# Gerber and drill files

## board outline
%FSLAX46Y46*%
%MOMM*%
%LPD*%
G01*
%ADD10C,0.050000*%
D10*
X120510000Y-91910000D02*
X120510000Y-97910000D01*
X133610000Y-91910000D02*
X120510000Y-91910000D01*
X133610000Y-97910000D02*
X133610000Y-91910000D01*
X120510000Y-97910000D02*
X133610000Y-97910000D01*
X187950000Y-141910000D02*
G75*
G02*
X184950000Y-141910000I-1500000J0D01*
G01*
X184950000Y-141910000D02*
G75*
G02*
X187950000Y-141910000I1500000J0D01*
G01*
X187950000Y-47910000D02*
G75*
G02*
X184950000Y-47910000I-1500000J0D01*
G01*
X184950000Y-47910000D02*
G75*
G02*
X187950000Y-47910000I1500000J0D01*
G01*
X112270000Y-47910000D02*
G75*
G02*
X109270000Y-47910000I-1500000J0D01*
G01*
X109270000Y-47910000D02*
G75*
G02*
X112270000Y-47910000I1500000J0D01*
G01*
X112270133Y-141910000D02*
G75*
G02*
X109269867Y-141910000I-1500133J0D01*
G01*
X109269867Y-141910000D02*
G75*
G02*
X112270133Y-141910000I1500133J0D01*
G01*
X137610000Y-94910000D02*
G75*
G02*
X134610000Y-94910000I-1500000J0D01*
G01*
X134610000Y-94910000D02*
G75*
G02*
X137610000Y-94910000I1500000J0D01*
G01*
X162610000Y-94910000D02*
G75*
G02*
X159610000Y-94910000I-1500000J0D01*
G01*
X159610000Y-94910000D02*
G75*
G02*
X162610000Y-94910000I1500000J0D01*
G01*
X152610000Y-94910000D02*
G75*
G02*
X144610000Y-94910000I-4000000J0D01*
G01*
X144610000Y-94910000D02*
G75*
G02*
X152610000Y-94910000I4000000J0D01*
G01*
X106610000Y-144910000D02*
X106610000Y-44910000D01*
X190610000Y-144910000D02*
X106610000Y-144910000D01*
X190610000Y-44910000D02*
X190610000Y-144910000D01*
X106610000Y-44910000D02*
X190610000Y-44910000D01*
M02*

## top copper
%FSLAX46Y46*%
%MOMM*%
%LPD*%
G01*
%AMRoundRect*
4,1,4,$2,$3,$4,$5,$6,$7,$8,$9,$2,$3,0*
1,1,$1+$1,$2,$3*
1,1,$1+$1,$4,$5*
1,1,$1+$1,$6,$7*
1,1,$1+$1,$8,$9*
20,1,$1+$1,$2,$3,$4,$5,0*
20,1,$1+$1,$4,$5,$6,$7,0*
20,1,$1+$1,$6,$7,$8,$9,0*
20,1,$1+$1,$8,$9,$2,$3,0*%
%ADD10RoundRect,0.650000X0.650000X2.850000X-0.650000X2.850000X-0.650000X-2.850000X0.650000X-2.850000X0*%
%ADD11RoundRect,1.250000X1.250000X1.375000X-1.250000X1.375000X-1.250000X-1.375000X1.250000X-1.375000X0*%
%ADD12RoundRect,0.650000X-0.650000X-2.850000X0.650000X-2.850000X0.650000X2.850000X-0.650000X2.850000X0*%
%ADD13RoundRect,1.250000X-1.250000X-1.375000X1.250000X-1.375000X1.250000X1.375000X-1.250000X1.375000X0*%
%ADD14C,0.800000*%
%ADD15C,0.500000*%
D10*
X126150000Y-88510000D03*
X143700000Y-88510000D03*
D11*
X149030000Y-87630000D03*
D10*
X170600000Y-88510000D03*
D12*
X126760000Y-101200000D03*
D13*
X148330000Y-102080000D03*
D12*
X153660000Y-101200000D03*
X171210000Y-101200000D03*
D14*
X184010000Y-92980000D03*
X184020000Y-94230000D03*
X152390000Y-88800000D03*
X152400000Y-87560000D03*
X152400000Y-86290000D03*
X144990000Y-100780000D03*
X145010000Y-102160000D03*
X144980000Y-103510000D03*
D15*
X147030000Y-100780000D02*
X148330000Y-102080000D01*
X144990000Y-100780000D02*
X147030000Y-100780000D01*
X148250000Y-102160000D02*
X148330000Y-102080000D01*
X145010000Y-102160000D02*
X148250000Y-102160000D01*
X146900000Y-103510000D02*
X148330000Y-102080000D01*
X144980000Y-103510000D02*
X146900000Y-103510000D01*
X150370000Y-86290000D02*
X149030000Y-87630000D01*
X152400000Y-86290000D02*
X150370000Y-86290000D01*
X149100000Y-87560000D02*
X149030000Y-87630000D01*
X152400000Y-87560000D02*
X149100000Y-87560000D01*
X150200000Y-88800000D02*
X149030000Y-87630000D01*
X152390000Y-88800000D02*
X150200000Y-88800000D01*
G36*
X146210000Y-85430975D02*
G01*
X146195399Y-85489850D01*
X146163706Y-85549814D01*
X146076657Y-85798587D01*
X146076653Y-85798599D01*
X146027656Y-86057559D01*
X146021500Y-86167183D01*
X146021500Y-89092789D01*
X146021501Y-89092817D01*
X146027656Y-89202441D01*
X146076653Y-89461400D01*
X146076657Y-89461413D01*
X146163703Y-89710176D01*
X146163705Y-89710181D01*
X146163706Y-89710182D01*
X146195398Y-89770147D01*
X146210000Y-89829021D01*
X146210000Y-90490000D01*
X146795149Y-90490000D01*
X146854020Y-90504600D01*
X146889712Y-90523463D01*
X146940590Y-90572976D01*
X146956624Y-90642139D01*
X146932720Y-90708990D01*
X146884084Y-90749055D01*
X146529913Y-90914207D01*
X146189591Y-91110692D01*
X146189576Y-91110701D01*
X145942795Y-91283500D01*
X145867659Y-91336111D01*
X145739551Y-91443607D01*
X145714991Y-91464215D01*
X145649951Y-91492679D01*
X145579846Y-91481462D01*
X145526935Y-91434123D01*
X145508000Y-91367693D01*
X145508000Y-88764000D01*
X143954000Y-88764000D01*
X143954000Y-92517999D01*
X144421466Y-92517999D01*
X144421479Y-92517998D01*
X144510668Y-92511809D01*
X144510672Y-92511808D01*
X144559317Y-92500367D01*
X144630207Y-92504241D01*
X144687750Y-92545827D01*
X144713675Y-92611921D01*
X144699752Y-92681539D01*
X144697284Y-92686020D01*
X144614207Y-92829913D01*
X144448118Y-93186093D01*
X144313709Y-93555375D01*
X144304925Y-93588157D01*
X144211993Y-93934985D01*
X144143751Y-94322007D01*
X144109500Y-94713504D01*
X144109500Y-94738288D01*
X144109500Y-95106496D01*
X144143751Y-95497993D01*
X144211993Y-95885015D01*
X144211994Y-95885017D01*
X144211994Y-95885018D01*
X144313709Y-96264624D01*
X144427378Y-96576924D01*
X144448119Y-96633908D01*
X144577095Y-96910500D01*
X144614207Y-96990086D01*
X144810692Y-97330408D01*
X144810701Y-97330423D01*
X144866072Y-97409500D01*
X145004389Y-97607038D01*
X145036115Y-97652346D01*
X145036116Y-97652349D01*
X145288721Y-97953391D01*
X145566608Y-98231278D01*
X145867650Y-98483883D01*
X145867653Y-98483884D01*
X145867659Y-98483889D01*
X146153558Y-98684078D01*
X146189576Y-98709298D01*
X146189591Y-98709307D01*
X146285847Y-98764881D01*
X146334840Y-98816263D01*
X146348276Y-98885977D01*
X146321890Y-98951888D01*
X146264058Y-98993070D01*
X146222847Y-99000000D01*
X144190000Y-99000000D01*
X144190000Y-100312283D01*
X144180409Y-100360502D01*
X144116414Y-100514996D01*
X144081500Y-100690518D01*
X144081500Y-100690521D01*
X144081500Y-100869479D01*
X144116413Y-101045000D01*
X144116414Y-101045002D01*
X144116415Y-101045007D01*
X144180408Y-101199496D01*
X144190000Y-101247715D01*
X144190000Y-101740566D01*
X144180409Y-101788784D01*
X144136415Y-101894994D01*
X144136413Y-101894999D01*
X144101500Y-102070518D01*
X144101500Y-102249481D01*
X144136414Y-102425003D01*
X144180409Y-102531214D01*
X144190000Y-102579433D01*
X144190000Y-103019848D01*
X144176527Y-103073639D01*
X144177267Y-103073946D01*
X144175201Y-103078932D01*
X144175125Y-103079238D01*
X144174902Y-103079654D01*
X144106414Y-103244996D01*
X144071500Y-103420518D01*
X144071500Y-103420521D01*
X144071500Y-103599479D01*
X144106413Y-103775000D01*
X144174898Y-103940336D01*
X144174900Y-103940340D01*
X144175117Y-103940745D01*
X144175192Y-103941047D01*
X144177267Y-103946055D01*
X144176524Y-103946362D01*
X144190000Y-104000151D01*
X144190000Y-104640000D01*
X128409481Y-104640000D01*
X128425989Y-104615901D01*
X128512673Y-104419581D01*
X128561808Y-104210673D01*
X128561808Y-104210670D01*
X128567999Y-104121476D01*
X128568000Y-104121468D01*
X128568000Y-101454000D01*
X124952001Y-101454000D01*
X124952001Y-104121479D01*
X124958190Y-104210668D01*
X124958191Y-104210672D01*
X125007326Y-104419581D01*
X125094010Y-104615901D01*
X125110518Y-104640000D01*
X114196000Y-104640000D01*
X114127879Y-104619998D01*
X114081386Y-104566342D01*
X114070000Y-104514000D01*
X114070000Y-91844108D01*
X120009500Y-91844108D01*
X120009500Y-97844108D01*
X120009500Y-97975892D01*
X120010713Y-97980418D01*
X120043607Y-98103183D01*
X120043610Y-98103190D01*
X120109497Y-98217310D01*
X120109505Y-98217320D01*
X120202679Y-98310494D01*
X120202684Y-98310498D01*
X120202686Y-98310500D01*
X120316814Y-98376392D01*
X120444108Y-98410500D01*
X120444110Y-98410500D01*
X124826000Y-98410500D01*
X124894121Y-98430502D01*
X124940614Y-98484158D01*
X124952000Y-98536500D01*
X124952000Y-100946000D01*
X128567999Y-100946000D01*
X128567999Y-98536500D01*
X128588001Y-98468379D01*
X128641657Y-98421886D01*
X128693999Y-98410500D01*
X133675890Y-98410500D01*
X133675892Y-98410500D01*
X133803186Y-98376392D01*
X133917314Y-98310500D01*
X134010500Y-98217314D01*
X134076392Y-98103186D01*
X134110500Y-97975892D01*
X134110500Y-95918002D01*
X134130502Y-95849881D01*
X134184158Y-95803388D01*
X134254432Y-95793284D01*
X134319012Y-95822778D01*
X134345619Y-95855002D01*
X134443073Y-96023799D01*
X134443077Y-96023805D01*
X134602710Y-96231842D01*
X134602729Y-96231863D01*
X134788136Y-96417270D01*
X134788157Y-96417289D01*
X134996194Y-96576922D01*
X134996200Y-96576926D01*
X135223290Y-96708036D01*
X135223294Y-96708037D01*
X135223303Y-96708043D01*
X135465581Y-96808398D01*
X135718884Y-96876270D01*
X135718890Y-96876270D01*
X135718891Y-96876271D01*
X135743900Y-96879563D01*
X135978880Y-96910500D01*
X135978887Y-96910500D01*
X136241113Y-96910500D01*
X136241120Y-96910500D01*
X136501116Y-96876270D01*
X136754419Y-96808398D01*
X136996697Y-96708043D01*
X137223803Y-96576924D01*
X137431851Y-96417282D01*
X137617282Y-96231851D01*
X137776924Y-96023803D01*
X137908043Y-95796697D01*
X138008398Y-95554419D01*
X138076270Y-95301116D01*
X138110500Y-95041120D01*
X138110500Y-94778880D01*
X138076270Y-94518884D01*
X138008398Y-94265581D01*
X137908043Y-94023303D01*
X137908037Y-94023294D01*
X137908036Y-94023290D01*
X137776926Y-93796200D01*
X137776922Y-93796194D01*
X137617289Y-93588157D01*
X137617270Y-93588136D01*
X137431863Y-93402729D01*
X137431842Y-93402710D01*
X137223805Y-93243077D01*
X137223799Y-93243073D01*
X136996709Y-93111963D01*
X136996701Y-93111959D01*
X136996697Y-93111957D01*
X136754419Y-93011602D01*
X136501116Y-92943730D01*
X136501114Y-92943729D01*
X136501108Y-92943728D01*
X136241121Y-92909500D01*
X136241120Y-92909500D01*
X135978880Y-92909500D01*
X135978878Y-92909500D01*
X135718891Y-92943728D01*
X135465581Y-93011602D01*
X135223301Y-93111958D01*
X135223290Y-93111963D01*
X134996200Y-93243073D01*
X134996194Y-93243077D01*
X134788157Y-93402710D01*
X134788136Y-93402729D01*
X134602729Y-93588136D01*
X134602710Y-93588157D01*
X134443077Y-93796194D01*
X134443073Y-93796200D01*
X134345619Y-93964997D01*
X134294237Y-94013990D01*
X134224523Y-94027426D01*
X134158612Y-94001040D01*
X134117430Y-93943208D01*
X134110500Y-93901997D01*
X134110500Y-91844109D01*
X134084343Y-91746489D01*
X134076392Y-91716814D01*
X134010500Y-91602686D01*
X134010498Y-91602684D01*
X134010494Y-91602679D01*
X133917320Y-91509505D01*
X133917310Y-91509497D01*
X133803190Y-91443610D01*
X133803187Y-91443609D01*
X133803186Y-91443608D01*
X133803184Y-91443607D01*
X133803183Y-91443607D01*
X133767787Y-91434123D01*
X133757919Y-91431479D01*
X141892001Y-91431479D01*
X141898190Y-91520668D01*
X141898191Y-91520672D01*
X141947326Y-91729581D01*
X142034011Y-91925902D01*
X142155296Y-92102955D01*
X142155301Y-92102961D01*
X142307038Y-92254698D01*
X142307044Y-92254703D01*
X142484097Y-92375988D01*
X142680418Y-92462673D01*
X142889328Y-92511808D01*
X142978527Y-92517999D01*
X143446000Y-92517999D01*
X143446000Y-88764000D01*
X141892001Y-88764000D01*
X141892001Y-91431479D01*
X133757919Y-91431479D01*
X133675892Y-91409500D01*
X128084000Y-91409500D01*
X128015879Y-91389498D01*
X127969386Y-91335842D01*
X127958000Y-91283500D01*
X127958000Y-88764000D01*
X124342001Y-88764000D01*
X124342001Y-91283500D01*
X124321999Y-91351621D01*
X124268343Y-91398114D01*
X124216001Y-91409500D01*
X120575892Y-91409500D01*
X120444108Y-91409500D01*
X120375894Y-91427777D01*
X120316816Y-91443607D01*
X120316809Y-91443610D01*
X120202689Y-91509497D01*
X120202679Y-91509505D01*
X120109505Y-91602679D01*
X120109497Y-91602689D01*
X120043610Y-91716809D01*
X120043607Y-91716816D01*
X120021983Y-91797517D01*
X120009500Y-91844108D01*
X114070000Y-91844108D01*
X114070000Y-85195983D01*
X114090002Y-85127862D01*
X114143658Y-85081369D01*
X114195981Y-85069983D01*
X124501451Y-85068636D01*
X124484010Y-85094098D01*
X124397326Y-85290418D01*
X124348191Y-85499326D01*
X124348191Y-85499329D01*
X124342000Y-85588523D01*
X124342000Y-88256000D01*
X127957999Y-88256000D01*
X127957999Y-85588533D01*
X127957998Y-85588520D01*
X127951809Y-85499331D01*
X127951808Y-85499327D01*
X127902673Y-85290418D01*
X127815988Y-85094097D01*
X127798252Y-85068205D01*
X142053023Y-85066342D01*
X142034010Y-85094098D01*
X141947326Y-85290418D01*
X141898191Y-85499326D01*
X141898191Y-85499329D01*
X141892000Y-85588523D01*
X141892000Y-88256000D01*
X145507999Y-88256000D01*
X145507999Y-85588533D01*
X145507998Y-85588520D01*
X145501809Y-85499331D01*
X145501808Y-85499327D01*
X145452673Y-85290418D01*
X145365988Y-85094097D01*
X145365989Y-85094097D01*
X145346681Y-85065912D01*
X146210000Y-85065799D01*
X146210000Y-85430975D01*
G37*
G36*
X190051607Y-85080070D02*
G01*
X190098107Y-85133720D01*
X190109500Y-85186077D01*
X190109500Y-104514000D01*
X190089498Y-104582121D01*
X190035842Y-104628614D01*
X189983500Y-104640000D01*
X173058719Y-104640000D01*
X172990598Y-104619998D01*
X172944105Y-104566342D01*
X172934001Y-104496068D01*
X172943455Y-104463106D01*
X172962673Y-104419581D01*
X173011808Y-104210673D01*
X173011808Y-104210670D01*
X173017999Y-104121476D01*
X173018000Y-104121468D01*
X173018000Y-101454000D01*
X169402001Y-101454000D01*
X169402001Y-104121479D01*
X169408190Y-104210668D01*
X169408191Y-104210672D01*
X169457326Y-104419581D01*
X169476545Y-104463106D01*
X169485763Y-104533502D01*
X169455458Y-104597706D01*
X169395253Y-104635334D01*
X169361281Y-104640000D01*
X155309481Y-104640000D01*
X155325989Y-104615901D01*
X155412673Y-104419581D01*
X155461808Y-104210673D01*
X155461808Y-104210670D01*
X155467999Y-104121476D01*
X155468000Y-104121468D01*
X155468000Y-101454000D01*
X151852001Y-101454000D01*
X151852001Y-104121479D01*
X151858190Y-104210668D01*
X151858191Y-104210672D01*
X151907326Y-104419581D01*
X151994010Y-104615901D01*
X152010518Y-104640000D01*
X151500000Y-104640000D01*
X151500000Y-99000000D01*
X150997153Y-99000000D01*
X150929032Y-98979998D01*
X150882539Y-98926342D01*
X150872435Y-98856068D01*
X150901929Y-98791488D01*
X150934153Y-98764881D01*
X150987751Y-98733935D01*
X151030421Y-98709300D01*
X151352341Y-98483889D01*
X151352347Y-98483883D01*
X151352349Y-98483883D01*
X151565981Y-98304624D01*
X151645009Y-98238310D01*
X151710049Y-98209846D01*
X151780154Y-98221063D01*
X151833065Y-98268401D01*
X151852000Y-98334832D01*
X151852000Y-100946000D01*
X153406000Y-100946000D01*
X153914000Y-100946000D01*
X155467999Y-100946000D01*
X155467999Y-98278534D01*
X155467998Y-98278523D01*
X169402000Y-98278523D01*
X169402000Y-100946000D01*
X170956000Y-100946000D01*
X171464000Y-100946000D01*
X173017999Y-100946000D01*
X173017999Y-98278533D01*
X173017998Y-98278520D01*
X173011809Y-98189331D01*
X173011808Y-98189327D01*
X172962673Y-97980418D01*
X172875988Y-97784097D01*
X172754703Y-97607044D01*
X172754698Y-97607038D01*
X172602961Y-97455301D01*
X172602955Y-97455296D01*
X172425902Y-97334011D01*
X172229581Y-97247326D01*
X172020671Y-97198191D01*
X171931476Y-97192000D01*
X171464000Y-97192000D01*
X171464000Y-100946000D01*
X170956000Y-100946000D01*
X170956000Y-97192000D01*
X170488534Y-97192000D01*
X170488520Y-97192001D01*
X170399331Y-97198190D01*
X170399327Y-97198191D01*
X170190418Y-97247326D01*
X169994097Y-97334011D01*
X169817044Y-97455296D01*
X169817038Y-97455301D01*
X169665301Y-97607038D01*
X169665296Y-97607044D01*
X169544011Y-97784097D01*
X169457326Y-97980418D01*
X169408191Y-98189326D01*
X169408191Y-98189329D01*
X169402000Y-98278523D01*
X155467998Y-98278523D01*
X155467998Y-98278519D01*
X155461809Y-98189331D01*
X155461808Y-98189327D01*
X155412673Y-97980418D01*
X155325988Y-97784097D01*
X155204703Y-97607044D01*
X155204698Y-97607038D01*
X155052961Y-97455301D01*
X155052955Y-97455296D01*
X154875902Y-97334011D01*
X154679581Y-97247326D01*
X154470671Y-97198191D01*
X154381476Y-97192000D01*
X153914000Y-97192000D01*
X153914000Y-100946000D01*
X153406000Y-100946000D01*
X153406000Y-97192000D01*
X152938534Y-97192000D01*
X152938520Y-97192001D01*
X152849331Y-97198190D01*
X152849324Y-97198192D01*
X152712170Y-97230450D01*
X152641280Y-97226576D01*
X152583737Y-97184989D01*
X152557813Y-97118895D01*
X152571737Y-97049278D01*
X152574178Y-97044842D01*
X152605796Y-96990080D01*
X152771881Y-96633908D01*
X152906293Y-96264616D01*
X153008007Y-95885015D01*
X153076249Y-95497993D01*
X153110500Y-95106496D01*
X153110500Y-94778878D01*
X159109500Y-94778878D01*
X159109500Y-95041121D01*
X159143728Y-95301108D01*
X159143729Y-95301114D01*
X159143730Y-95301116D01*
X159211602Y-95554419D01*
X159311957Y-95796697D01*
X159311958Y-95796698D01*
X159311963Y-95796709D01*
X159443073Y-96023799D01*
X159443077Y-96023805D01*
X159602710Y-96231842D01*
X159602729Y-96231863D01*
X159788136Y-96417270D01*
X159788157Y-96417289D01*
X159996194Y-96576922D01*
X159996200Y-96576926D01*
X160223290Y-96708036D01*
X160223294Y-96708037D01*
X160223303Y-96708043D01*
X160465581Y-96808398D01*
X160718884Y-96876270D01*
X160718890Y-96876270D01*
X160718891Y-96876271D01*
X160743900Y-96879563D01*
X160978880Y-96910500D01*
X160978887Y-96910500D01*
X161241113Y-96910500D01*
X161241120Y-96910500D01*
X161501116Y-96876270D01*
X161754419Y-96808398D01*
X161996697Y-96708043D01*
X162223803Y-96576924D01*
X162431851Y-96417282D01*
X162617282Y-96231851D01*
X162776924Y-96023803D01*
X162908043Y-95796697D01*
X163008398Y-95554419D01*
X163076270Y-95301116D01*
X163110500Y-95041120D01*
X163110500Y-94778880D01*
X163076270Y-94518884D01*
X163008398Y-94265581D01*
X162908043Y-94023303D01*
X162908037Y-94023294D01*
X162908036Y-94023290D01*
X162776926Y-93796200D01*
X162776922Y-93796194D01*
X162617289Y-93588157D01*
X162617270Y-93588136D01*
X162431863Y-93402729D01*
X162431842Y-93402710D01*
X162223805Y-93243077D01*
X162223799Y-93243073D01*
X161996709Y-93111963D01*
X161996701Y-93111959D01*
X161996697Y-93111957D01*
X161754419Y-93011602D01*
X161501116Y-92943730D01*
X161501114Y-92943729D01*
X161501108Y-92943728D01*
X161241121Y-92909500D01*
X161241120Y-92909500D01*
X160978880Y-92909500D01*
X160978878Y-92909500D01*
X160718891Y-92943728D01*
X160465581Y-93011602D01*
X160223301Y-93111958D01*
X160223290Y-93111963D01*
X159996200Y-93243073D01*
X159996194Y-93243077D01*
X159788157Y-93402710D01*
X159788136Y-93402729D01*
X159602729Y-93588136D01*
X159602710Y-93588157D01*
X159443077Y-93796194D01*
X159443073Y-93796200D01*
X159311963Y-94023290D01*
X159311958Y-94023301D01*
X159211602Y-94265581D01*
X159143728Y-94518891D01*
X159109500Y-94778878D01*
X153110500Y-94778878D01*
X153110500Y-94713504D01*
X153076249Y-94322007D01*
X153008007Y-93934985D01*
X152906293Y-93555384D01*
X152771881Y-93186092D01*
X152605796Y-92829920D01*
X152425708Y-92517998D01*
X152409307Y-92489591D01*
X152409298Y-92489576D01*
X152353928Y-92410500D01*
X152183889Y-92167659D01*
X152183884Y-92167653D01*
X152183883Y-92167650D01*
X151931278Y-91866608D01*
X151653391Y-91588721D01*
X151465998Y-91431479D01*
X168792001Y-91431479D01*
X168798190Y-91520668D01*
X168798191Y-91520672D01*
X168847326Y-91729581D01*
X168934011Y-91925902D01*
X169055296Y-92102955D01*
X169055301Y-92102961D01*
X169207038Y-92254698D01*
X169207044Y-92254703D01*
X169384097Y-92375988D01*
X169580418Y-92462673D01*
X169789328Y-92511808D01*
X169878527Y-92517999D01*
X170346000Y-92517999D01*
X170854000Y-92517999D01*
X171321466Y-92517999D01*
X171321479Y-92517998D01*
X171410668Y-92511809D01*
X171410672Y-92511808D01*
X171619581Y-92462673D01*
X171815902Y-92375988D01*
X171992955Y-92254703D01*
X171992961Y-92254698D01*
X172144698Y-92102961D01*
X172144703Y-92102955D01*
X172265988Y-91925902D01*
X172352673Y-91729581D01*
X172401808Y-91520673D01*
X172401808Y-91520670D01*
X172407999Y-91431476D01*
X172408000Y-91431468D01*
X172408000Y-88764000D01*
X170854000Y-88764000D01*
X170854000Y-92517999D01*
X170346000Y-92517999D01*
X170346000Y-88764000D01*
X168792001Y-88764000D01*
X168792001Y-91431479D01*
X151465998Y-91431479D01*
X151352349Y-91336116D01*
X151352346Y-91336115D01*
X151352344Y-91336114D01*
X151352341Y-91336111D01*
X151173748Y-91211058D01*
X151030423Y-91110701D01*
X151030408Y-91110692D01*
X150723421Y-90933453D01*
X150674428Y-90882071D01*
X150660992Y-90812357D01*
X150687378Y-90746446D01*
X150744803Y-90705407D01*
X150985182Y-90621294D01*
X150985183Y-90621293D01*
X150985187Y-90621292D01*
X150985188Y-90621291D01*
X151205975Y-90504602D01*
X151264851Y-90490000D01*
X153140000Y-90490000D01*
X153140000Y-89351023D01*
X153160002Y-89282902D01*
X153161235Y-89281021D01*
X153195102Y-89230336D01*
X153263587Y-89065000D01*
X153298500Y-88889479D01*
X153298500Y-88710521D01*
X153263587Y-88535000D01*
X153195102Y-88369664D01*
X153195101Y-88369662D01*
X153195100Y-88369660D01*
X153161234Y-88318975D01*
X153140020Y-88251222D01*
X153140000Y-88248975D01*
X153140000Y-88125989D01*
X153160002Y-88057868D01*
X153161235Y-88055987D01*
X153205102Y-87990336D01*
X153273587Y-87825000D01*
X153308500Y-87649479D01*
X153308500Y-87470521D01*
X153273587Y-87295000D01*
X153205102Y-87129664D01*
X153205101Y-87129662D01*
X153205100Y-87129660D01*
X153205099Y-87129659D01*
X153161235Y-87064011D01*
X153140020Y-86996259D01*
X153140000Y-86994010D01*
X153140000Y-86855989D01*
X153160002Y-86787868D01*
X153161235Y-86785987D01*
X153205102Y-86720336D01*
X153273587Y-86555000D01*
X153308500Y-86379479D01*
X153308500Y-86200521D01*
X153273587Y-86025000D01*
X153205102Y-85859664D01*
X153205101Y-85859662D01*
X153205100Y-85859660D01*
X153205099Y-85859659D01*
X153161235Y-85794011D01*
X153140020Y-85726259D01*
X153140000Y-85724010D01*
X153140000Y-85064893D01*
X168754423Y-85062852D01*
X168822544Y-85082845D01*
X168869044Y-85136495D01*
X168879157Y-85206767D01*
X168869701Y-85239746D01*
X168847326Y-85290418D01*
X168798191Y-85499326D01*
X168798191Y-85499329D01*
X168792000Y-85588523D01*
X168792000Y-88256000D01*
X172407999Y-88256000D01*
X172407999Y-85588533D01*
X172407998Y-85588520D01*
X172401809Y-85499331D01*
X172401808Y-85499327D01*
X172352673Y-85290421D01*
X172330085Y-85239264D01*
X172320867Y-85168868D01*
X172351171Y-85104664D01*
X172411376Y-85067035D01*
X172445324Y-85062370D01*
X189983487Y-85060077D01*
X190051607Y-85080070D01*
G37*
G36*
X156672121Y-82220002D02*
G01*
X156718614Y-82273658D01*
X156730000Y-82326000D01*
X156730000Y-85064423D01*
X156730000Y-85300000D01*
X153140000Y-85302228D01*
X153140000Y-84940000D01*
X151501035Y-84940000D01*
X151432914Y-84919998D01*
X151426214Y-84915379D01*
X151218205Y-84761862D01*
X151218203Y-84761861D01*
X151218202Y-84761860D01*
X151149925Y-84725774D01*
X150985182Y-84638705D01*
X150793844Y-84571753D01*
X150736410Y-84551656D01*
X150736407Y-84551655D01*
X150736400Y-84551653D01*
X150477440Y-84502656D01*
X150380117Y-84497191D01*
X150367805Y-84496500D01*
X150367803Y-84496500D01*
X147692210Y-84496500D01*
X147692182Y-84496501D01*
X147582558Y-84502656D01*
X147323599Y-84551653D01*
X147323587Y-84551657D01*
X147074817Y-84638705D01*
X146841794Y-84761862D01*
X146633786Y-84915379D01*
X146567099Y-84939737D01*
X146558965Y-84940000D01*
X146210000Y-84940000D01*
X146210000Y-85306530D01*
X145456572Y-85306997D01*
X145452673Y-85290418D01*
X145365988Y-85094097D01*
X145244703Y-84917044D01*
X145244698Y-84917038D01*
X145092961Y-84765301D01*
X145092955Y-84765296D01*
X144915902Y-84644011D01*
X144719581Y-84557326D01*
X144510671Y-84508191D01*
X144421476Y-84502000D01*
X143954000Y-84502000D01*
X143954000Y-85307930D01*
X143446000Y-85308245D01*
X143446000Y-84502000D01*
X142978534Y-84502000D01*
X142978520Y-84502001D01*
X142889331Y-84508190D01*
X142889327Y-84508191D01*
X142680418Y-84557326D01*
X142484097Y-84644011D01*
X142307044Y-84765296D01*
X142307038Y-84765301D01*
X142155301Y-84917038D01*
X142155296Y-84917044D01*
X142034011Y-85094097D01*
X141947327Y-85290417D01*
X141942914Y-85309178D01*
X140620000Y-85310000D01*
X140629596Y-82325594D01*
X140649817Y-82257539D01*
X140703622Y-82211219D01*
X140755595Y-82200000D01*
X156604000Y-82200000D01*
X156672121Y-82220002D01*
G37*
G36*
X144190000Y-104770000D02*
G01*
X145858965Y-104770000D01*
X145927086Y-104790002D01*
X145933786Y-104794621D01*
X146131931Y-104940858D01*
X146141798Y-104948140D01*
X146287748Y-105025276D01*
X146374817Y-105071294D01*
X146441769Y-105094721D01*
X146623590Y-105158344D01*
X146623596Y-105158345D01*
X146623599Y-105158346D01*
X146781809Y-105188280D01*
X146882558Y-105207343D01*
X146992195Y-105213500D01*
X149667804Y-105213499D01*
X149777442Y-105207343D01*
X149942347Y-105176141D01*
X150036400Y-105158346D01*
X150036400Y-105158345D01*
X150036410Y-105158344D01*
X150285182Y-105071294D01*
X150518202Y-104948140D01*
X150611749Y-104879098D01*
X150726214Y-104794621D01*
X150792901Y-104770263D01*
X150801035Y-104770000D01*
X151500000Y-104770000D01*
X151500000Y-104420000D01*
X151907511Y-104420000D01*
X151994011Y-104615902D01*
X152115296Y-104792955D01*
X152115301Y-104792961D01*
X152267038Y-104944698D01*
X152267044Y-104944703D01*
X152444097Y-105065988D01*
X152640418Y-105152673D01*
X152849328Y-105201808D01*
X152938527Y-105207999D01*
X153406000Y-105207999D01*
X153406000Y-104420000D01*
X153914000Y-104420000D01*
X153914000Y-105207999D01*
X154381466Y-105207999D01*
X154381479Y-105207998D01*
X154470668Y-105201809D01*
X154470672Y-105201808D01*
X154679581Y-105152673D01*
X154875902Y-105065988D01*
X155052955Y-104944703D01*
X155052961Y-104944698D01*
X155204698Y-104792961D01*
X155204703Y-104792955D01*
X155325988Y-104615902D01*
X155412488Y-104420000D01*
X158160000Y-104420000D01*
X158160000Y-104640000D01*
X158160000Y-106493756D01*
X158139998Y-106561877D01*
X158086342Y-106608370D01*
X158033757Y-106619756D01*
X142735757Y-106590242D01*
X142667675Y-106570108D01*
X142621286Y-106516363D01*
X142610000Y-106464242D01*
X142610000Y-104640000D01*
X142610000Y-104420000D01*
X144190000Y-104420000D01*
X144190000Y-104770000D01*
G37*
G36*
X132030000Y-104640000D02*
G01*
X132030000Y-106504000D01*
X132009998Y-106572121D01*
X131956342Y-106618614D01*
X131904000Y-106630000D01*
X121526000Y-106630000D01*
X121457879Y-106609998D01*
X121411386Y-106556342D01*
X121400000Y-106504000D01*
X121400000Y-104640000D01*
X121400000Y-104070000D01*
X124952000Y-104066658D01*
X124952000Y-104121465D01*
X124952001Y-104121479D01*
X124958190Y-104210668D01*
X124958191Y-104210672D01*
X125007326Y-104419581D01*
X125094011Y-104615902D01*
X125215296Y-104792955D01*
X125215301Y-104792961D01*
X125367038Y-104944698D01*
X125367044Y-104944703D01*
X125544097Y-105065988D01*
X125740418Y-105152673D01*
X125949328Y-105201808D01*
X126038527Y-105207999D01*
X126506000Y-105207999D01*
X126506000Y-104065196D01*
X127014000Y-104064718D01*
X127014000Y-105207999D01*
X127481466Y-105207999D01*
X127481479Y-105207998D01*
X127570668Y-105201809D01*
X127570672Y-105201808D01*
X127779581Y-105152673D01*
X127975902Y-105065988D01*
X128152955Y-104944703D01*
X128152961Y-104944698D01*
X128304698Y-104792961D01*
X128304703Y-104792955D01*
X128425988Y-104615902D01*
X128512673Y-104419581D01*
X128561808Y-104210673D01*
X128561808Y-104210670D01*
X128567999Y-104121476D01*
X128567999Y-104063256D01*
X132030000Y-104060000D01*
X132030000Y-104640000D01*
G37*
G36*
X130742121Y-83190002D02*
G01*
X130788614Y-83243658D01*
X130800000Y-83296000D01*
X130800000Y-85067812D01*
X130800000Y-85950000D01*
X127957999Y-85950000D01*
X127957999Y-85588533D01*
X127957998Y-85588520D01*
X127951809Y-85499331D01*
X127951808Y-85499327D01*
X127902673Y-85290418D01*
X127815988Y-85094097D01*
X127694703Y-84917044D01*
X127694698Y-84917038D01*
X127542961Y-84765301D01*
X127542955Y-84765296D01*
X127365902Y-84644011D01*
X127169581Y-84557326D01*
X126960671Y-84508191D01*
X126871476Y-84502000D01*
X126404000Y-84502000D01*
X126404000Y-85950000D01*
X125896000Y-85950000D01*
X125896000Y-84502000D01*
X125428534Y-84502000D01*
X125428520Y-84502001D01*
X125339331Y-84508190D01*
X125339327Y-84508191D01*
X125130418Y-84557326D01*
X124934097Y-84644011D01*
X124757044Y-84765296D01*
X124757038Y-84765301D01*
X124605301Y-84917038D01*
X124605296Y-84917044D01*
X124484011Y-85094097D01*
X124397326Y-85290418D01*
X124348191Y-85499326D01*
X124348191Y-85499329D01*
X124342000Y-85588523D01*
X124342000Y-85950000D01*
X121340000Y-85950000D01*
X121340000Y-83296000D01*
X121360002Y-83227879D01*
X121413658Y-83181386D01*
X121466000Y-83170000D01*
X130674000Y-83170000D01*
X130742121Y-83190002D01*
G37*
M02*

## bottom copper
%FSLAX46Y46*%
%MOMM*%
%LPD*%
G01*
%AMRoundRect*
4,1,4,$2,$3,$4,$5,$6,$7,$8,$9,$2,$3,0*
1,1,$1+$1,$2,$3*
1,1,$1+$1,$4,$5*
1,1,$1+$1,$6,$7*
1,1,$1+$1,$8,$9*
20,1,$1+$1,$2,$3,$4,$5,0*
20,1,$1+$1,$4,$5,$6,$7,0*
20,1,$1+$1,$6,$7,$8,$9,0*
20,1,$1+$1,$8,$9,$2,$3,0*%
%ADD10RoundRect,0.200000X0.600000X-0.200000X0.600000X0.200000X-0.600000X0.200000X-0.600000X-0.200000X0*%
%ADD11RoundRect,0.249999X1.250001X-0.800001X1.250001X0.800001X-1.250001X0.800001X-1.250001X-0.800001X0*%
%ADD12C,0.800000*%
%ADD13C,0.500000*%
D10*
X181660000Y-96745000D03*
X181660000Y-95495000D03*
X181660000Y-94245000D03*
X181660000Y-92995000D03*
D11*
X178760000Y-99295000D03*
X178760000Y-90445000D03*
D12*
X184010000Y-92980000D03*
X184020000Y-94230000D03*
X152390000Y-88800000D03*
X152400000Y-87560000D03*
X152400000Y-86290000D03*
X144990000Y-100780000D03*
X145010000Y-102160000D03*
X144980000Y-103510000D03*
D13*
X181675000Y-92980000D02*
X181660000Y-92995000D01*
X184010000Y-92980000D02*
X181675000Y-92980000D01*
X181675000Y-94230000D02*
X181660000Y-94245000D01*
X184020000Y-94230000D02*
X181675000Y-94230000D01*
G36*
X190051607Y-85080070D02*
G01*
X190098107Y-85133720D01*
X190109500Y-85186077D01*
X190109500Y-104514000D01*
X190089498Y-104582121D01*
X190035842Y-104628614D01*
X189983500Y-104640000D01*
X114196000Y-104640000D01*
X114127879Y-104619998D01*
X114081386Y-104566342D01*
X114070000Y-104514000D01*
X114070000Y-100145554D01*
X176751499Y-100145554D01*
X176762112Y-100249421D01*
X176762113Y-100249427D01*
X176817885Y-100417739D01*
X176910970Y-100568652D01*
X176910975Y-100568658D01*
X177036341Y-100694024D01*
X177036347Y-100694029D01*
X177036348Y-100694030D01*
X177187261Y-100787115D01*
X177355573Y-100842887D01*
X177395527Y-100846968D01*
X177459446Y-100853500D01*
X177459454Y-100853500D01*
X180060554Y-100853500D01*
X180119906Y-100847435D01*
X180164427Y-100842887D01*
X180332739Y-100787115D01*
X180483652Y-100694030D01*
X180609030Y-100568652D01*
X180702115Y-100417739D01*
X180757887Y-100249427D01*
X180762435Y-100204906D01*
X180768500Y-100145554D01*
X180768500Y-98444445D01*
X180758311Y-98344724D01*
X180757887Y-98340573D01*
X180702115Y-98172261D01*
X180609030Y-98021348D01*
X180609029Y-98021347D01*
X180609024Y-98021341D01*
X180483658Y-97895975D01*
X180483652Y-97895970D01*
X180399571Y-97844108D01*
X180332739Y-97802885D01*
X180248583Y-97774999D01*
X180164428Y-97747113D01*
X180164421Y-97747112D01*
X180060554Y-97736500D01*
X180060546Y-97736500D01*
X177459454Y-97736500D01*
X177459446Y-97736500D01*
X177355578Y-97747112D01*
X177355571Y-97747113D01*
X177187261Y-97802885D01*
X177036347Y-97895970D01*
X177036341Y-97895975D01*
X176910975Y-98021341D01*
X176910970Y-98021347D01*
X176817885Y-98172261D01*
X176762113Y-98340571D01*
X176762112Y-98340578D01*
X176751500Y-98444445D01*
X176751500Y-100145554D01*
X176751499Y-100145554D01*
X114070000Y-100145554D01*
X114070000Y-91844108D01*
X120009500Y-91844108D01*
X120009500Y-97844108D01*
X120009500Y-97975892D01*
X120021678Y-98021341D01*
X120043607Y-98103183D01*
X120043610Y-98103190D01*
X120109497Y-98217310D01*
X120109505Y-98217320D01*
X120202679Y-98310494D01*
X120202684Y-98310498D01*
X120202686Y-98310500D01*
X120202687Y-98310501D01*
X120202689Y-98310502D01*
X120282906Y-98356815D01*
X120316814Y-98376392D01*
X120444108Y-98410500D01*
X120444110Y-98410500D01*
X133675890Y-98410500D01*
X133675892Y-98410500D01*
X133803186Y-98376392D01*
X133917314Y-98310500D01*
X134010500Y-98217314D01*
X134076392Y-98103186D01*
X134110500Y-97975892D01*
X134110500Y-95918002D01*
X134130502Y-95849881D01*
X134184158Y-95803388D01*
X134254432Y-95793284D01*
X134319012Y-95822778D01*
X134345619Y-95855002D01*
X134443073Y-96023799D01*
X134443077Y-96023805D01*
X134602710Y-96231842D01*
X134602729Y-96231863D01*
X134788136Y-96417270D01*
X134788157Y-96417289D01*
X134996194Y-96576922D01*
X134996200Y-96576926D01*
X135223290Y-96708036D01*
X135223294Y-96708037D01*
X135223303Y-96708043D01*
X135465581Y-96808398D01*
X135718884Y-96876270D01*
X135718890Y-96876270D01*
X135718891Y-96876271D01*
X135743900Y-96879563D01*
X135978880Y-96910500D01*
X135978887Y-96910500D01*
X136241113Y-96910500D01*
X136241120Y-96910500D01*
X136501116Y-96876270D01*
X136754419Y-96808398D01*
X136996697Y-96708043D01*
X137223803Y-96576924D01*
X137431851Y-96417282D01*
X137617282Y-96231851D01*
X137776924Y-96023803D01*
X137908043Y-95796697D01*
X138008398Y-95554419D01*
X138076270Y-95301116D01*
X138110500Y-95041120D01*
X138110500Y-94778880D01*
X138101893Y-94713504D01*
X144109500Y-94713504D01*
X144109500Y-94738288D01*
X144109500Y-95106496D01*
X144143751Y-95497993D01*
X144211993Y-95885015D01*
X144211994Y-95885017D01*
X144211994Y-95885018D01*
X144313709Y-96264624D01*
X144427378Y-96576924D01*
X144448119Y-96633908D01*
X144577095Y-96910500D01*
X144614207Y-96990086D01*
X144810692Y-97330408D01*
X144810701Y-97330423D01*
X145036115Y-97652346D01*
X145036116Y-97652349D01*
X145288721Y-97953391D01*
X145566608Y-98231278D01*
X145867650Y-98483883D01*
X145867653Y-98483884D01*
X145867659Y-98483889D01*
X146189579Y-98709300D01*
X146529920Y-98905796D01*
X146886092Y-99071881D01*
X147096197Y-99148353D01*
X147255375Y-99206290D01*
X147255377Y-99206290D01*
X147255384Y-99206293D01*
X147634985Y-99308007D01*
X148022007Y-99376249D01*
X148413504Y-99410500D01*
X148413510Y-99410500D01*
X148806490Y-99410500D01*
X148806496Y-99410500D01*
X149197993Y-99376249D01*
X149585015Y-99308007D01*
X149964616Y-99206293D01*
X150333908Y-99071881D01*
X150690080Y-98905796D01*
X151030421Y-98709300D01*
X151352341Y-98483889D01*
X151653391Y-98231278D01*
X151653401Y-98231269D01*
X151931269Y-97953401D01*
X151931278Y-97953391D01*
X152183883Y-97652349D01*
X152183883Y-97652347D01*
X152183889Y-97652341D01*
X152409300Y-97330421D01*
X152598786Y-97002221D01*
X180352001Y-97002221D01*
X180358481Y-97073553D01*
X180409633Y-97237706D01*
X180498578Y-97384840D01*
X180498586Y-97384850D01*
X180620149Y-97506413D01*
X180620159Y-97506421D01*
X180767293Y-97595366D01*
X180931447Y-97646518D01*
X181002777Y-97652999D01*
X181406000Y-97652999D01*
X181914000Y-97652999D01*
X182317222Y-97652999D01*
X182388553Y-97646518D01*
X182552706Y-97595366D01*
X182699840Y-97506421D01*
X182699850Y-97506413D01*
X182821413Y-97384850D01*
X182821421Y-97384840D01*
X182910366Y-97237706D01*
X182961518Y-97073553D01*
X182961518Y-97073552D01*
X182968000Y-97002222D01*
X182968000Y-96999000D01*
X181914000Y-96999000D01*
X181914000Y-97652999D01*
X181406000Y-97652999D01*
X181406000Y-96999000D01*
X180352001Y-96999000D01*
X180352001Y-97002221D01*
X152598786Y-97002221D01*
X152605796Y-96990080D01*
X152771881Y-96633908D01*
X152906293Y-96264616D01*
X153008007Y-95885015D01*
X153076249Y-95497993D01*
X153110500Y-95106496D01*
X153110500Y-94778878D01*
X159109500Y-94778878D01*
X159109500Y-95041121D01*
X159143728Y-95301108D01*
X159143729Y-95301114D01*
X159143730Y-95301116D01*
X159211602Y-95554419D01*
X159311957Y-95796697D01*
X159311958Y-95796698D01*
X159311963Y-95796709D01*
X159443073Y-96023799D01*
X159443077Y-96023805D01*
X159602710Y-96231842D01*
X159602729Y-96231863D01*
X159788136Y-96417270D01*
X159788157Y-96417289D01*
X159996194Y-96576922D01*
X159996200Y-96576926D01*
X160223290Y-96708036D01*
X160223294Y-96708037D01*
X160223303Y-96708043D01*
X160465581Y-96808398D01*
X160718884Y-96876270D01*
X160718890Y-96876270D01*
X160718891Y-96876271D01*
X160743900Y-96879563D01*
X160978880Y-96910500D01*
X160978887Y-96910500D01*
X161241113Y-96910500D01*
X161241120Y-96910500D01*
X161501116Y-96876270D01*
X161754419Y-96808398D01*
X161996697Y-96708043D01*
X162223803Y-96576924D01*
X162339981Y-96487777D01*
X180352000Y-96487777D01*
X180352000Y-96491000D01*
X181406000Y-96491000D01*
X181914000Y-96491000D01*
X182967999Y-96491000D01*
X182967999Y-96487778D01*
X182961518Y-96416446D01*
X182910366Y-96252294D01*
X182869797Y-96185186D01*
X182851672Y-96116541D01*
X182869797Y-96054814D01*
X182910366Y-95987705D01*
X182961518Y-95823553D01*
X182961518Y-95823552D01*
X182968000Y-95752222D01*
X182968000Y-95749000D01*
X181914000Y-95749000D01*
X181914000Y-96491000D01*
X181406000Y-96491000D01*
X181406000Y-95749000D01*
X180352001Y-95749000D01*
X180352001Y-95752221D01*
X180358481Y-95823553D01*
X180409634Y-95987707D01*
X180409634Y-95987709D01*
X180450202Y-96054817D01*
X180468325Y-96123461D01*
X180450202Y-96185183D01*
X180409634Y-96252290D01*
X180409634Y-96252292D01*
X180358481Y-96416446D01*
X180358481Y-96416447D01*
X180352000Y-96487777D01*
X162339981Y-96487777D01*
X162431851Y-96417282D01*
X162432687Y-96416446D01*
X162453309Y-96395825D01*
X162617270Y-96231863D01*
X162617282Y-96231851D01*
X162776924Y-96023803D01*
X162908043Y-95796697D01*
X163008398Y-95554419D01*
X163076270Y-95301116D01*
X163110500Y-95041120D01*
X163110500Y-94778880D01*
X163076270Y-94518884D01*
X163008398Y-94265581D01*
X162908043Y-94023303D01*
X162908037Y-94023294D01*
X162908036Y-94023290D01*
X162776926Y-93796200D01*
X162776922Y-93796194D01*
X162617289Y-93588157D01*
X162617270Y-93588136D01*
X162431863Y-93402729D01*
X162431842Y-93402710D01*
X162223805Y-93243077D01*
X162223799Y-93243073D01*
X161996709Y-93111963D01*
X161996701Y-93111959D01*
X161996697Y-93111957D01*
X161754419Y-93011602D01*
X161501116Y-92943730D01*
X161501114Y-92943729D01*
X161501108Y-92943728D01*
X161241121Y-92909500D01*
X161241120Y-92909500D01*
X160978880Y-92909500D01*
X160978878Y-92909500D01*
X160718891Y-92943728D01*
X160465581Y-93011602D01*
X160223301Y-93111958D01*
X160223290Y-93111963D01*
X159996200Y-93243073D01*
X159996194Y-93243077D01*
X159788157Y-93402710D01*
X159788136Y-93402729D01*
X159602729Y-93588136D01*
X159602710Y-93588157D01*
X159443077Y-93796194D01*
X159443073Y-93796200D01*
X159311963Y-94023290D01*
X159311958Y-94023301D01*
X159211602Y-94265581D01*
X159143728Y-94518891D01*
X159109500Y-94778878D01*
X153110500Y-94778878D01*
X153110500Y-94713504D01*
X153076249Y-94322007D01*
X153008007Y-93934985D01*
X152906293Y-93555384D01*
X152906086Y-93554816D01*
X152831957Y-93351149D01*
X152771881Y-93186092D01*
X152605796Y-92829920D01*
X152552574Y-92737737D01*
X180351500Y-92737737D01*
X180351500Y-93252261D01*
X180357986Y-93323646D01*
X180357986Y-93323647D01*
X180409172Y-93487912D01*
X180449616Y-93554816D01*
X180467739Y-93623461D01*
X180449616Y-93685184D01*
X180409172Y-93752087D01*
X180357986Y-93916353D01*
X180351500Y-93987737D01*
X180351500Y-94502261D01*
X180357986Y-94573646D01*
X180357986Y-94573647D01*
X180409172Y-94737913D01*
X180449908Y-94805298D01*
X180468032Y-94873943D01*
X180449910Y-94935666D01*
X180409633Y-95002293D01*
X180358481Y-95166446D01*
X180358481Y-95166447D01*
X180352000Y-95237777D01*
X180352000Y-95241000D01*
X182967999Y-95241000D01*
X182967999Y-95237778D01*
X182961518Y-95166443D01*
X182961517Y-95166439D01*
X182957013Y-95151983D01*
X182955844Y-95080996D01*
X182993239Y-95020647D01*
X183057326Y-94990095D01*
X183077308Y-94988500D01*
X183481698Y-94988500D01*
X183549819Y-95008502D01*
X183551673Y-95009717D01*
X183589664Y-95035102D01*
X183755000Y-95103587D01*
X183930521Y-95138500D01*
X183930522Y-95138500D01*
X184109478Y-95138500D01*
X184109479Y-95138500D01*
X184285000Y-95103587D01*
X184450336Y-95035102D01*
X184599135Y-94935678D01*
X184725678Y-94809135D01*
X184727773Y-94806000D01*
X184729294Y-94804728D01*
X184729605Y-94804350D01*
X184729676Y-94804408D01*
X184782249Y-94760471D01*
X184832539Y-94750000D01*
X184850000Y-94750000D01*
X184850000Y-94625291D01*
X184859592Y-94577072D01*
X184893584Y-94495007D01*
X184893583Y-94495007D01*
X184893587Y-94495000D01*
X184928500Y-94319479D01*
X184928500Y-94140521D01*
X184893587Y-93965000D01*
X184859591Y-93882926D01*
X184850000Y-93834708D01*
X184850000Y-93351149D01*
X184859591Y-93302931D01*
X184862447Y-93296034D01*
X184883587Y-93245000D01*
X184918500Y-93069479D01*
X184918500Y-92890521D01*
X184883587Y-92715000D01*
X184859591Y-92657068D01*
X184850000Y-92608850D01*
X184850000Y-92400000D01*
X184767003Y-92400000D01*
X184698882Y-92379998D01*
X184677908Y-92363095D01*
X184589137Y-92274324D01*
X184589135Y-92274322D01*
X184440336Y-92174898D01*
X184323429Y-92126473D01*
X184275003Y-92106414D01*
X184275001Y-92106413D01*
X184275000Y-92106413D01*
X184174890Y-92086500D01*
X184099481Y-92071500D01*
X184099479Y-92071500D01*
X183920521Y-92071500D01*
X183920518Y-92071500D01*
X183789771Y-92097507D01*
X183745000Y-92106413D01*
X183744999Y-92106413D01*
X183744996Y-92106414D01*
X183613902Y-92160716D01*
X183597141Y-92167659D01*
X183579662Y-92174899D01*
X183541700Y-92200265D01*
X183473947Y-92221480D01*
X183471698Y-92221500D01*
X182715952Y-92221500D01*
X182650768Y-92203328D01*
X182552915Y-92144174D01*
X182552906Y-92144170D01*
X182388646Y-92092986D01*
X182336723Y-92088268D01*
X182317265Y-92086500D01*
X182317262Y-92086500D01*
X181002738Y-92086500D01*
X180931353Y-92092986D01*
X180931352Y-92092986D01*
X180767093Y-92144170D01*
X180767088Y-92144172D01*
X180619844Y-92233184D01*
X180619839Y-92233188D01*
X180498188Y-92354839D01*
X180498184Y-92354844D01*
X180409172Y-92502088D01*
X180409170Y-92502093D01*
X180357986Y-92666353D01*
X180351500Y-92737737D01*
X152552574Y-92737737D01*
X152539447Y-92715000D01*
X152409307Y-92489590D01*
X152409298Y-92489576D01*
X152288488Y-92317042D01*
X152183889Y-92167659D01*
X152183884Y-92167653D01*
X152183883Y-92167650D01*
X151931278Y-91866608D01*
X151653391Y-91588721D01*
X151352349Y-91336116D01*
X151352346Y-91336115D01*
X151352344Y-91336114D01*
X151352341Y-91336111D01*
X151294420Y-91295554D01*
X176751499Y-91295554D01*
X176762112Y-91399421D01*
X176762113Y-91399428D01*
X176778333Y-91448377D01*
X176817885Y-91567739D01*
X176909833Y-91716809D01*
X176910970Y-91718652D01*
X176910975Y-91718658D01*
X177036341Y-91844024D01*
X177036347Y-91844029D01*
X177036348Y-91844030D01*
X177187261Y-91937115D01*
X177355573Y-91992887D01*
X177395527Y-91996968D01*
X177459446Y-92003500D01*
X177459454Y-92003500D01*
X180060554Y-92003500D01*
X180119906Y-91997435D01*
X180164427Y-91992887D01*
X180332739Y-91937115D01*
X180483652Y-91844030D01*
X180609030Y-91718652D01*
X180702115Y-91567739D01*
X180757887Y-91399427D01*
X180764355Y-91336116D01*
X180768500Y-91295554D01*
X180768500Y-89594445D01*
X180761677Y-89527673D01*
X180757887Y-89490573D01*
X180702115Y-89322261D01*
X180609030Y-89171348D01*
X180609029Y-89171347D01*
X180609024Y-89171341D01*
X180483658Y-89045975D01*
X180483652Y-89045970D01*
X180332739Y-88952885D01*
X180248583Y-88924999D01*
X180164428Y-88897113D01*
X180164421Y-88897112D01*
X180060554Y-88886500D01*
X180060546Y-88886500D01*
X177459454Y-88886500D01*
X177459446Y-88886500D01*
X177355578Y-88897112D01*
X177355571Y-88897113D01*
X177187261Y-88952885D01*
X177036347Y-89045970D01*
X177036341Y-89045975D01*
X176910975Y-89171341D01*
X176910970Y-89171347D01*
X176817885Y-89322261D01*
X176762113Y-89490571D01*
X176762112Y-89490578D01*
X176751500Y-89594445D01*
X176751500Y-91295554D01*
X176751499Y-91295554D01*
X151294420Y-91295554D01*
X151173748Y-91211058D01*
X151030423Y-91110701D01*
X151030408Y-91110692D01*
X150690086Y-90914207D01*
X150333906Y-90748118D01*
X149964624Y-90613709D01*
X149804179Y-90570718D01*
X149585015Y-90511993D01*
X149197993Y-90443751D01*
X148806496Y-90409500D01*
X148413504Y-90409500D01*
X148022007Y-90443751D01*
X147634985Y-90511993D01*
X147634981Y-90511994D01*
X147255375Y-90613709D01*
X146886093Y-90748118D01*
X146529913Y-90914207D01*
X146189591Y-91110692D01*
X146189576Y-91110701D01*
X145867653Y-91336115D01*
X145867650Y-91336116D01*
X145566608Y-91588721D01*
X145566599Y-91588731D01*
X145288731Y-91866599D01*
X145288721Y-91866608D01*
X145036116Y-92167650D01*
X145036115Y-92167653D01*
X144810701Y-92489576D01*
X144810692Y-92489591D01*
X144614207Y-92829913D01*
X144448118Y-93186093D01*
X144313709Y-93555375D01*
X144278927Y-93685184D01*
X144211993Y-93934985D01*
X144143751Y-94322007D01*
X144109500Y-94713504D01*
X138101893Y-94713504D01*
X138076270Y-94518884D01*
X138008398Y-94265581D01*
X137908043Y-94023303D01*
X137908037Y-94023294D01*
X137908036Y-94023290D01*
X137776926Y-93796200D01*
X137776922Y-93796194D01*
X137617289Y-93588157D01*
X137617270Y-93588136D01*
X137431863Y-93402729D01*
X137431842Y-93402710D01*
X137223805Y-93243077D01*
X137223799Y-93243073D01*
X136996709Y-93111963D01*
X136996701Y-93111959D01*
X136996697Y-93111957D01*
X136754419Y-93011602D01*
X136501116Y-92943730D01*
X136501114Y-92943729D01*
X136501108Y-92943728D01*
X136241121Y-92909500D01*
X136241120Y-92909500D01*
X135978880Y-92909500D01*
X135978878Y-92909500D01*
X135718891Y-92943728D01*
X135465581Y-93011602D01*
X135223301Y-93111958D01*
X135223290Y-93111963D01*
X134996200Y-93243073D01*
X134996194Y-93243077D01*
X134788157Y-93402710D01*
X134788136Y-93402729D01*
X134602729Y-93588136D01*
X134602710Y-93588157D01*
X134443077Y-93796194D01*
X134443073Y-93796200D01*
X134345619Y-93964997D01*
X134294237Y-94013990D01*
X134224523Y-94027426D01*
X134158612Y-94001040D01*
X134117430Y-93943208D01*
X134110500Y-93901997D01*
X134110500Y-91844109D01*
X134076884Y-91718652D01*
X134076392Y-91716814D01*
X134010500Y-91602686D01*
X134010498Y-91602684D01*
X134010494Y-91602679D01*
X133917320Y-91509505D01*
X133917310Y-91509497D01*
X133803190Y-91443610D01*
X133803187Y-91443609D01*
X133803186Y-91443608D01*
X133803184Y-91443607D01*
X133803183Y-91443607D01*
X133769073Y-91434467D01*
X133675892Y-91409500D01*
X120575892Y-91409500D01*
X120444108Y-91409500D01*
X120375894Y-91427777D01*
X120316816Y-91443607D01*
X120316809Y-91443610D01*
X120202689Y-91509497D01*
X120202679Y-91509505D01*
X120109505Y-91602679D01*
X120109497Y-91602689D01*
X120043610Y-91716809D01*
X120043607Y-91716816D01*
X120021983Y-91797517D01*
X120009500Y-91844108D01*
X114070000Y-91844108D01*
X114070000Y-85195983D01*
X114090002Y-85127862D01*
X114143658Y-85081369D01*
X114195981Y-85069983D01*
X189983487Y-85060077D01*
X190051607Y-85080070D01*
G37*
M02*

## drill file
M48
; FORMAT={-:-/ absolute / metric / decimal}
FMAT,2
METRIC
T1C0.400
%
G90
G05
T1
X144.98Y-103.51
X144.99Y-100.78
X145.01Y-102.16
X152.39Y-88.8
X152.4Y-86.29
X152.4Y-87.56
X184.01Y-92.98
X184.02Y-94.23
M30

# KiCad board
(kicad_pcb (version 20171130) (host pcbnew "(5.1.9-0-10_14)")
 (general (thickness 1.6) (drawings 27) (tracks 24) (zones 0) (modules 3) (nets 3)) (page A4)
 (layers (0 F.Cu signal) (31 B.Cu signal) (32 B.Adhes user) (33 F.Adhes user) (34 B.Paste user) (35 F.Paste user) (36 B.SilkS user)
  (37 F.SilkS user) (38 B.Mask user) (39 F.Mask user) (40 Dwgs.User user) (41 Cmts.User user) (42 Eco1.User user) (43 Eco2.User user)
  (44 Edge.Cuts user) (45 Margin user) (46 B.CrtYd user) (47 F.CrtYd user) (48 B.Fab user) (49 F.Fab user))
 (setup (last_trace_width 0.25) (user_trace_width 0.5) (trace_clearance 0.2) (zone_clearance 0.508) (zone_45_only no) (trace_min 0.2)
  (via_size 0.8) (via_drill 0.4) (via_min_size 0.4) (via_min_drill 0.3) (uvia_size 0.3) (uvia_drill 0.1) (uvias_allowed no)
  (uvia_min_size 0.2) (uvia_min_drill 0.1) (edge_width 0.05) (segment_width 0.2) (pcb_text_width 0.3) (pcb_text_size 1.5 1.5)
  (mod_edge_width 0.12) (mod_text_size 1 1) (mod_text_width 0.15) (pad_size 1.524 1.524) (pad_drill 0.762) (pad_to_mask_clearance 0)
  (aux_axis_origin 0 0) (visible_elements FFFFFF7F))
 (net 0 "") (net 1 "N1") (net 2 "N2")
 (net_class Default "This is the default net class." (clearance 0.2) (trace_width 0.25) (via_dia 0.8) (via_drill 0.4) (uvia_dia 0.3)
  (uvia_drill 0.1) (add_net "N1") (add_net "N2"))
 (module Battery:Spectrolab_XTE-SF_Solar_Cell (layer F.Cu) (at 183.23 85.01 180)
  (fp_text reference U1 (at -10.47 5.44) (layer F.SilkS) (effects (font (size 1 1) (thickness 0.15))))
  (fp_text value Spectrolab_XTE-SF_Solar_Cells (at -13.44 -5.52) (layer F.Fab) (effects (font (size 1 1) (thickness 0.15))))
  (pad 4 smd roundrect (at 57.08 -3.5 180) (size 2.6 7) (layers F.Cu F.Paste F.Mask) (roundrect_rratio 0.25) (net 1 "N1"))
  (pad 3 smd roundrect (at 39.53 -3.5 180) (size 2.6 7) (layers F.Cu F.Paste F.Mask) (roundrect_rratio 0.25) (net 1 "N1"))
  (pad 2 smd roundrect (at 34.2 -2.62 180) (size 5 5.25) (layers F.Cu F.Paste F.Mask) (roundrect_rratio 0.25) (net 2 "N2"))
  (pad 1 smd roundrect (at 12.63 -3.5 180) (size 2.6 7) (layers F.Cu F.Paste F.Mask) (roundrect_rratio 0.25) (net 1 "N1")))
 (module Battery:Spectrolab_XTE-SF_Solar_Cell (layer F.Cu) (at 114.13 104.7)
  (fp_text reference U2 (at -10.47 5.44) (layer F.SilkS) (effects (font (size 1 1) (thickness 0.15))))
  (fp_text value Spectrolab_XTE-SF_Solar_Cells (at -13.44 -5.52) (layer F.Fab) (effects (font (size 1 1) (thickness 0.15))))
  (pad 1 smd roundrect (at 12.63 -3.5) (size 2.6 7) (layers F.Cu F.Paste F.Mask) (roundrect_rratio 0.25) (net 1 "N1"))
  (pad 2 smd roundrect (at 34.2 -2.62) (size 5 5.25) (layers F.Cu F.Paste F.Mask) (roundrect_rratio 0.25) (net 2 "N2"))
  (pad 3 smd roundrect (at 39.53 -3.5) (size 2.6 7) (layers F.Cu F.Paste F.Mask) (roundrect_rratio 0.25) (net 1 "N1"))
  (pad 4 smd roundrect (at 57.08 -3.5) (size 2.6 7) (layers F.Cu F.Paste F.Mask) (roundrect_rratio 0.25) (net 1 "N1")))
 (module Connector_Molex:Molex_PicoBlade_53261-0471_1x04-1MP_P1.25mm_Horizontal (layer B.Cu) (at 179.26 94.87 90)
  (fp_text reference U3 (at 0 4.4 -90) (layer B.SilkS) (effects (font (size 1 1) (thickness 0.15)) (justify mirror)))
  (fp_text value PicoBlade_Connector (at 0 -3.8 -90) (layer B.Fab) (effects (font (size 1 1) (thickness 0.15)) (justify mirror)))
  (pad 1 smd roundrect (at -1.875 2.4 90) (size 0.8 1.6) (layers B.Cu B.Paste B.Mask) (roundrect_rratio 0.25) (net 2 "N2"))
  (pad 2 smd roundrect (at -0.625 2.4 90) (size 0.8 1.6) (layers B.Cu B.Paste B.Mask) (roundrect_rratio 0.25) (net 2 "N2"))
  (pad 3 smd roundrect (at 0.625 2.4 90) (size 0.8 1.6) (layers B.Cu B.Paste B.Mask) (roundrect_rratio 0.25) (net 1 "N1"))
  (pad 4 smd roundrect (at 1.875 2.4 90) (size 0.8 1.6) (layers B.Cu B.Paste B.Mask) (roundrect_rratio 0.25) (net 1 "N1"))
  (pad MP smd roundrect (at -4.425 -0.5 90) (size 2.1 3) (layers B.Cu B.Paste B.Mask) (roundrect_rratio 0.1190471428571429))
  (pad MP smd roundrect (at 4.425 -0.5 90) (size 2.1 3) (layers B.Cu B.Paste B.Mask) (roundrect_rratio 0.1190471428571429)))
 (gr_line (start 120.51 91.91) (end 120.51 97.91) (layer Edge.Cuts) (width 0.05))
 (gr_line (start 133.61 91.91) (end 120.51 91.91) (layer Edge.Cuts) (width 0.05))
 (gr_line (start 133.61 97.91) (end 133.61 91.91) (layer Edge.Cuts) (width 0.05))
 (gr_line (start 120.51 97.91) (end 133.61 97.91) (layer Edge.Cuts) (width 0.05))
 (gr_circle (center 186.45 141.91) (end 187.95 141.91) (layer Edge.Cuts) (width 0.05))
 (gr_circle (center 186.45 47.91) (end 187.95 47.91) (layer Edge.Cuts) (width 0.05))
 (gr_circle (center 110.77 47.91) (end 112.27 47.91) (layer Edge.Cuts) (width 0.05))
 (gr_circle (center 110.77 141.91) (end 112.27 141.89) (layer Edge.Cuts) (width 0.05))
 (gr_circle (center 136.11 94.91) (end 137.61 94.91) (layer Edge.Cuts) (width 0.05))
 (gr_circle (center 161.11 94.91) (end 162.61 94.91) (layer Edge.Cuts) (width 0.05))
 (gr_circle (center 148.61 94.91) (end 152.61 94.91) (layer Edge.Cuts) (width 0.05))
 (gr_line (start 106.61 144.91) (end 106.61 44.91) (layer Edge.Cuts) (width 0.05))
 (gr_line (start 190.61 144.91) (end 106.61 144.91) (layer Edge.Cuts) (width 0.05))
 (gr_line (start 190.61 44.91) (end 190.61 144.91) (layer Edge.Cuts) (width 0.05))
 (gr_line (start 106.61 44.91) (end 190.61 44.91) (layer Edge.Cuts) (width 0.05))
 (via (at 184.01 92.98) (size 0.8) (drill 0.4) (layers F.Cu B.Cu) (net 1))
 (via (at 184.02 94.23) (size 0.8) (drill 0.4) (layers F.Cu B.Cu) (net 1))
 (segment (start 181.675 92.98) (end 181.66 92.995) (width 0.5) (layer B.Cu) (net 1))
 (segment (start 184.01 92.98) (end 181.675 92.98) (width 0.5) (layer B.Cu) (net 1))
 (segment (start 181.675 94.23) (end 181.66 94.245) (width 0.5) (layer B.Cu) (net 1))
 (segment (start 184.02 94.23) (end 181.675 94.23) (width 0.5) (layer B.Cu) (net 1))
 (via (at 152.39 88.8) (size 0.8) (drill 0.4) (layers F.Cu B.Cu) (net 2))
 (via (at 152.4 87.56) (size 0.8) (drill 0.4) (layers F.Cu B.Cu) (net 2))
 (via (at 152.4 86.29) (size 0.8) (drill 0.4) (layers F.Cu B.Cu) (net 2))
 (via (at 144.99 100.78) (size 0.8) (drill 0.4) (layers F.Cu B.Cu) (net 2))
 (via (at 145.01 102.16) (size 0.8) (drill 0.4) (layers F.Cu B.Cu) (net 2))
 (via (at 144.98 103.51) (size 0.8) (drill 0.4) (layers F.Cu B.Cu) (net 2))
 (segment (start 147.03 100.78) (end 148.33 102.08) (width 0.5) (layer F.Cu) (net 2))
 (segment (start 144.99 100.78) (end 147.03 100.78) (width 0.5) (layer F.Cu) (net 2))
 (segment (start 148.25 102.16) (end 148.33 102.08) (width 0.5) (layer F.Cu) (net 2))
 (segment (start 145.01 102.16) (end 148.25 102.16) (width 0.5) (layer F.Cu) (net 2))
 (segment (start 146.9 103.51) (end 148.33 102.08) (width 0.5) (layer F.Cu) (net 2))
 (segment (start 144.98 103.51) (end 146.9 103.51) (width 0.5) (layer F.Cu) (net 2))
 (segment (start 150.37 86.29) (end 149.03 87.63) (width 0.5) (layer F.Cu) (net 2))
 (segment (start 152.4 86.29) (end 150.37 86.29) (width 0.5) (layer F.Cu) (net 2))
 (segment (start 149.1 87.56) (end 149.03 87.63) (width 0.5) (layer F.Cu) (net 2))
 (segment (start 152.4 87.56) (end 149.1 87.56) (width 0.5) (layer F.Cu) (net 2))
 (segment (start 150.2 88.8) (end 149.03 87.63) (width 0.5) (layer F.Cu) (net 2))
 (segment (start 152.39 88.8) (end 150.2 88.8) (width 0.5) (layer F.Cu) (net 2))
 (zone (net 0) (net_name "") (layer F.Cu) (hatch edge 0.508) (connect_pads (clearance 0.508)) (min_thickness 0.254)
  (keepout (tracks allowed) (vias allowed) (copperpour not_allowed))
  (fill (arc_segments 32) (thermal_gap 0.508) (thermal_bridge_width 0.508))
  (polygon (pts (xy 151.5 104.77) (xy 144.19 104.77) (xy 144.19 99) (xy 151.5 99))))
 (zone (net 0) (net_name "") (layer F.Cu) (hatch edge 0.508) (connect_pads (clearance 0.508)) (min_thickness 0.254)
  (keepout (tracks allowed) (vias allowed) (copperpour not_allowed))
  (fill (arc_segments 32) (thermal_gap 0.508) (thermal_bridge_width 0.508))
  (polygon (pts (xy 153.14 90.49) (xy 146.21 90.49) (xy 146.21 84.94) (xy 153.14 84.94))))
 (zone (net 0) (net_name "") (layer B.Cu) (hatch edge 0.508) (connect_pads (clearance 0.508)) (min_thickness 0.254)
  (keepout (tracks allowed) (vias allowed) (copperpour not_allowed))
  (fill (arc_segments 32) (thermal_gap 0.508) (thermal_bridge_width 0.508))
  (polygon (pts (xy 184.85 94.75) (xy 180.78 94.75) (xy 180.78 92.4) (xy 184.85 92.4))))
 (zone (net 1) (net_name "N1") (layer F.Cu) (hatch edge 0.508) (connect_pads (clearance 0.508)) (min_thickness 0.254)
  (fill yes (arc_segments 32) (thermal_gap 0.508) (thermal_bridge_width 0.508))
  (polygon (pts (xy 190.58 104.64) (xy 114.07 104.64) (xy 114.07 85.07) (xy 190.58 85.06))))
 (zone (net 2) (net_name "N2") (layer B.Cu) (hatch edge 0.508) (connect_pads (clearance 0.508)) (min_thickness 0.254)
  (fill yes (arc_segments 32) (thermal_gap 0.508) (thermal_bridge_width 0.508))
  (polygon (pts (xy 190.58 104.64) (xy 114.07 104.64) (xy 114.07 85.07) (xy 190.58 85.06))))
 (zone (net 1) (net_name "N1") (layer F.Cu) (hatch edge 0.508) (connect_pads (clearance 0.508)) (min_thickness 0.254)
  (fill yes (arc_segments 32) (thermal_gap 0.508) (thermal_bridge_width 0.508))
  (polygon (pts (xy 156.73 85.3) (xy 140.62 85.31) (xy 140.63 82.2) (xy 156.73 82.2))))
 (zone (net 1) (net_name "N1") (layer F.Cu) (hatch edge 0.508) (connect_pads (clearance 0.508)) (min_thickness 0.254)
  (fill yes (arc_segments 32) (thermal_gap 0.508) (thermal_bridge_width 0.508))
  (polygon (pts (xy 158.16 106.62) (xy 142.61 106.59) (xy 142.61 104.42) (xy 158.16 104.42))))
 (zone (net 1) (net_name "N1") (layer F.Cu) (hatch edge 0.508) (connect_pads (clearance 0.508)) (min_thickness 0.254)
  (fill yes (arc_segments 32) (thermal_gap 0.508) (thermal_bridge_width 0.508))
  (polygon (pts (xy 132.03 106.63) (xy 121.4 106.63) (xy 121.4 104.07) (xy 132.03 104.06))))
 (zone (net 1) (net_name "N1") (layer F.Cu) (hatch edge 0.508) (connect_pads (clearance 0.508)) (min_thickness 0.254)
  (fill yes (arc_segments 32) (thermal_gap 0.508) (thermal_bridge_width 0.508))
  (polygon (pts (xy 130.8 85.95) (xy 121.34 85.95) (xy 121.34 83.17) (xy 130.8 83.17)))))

